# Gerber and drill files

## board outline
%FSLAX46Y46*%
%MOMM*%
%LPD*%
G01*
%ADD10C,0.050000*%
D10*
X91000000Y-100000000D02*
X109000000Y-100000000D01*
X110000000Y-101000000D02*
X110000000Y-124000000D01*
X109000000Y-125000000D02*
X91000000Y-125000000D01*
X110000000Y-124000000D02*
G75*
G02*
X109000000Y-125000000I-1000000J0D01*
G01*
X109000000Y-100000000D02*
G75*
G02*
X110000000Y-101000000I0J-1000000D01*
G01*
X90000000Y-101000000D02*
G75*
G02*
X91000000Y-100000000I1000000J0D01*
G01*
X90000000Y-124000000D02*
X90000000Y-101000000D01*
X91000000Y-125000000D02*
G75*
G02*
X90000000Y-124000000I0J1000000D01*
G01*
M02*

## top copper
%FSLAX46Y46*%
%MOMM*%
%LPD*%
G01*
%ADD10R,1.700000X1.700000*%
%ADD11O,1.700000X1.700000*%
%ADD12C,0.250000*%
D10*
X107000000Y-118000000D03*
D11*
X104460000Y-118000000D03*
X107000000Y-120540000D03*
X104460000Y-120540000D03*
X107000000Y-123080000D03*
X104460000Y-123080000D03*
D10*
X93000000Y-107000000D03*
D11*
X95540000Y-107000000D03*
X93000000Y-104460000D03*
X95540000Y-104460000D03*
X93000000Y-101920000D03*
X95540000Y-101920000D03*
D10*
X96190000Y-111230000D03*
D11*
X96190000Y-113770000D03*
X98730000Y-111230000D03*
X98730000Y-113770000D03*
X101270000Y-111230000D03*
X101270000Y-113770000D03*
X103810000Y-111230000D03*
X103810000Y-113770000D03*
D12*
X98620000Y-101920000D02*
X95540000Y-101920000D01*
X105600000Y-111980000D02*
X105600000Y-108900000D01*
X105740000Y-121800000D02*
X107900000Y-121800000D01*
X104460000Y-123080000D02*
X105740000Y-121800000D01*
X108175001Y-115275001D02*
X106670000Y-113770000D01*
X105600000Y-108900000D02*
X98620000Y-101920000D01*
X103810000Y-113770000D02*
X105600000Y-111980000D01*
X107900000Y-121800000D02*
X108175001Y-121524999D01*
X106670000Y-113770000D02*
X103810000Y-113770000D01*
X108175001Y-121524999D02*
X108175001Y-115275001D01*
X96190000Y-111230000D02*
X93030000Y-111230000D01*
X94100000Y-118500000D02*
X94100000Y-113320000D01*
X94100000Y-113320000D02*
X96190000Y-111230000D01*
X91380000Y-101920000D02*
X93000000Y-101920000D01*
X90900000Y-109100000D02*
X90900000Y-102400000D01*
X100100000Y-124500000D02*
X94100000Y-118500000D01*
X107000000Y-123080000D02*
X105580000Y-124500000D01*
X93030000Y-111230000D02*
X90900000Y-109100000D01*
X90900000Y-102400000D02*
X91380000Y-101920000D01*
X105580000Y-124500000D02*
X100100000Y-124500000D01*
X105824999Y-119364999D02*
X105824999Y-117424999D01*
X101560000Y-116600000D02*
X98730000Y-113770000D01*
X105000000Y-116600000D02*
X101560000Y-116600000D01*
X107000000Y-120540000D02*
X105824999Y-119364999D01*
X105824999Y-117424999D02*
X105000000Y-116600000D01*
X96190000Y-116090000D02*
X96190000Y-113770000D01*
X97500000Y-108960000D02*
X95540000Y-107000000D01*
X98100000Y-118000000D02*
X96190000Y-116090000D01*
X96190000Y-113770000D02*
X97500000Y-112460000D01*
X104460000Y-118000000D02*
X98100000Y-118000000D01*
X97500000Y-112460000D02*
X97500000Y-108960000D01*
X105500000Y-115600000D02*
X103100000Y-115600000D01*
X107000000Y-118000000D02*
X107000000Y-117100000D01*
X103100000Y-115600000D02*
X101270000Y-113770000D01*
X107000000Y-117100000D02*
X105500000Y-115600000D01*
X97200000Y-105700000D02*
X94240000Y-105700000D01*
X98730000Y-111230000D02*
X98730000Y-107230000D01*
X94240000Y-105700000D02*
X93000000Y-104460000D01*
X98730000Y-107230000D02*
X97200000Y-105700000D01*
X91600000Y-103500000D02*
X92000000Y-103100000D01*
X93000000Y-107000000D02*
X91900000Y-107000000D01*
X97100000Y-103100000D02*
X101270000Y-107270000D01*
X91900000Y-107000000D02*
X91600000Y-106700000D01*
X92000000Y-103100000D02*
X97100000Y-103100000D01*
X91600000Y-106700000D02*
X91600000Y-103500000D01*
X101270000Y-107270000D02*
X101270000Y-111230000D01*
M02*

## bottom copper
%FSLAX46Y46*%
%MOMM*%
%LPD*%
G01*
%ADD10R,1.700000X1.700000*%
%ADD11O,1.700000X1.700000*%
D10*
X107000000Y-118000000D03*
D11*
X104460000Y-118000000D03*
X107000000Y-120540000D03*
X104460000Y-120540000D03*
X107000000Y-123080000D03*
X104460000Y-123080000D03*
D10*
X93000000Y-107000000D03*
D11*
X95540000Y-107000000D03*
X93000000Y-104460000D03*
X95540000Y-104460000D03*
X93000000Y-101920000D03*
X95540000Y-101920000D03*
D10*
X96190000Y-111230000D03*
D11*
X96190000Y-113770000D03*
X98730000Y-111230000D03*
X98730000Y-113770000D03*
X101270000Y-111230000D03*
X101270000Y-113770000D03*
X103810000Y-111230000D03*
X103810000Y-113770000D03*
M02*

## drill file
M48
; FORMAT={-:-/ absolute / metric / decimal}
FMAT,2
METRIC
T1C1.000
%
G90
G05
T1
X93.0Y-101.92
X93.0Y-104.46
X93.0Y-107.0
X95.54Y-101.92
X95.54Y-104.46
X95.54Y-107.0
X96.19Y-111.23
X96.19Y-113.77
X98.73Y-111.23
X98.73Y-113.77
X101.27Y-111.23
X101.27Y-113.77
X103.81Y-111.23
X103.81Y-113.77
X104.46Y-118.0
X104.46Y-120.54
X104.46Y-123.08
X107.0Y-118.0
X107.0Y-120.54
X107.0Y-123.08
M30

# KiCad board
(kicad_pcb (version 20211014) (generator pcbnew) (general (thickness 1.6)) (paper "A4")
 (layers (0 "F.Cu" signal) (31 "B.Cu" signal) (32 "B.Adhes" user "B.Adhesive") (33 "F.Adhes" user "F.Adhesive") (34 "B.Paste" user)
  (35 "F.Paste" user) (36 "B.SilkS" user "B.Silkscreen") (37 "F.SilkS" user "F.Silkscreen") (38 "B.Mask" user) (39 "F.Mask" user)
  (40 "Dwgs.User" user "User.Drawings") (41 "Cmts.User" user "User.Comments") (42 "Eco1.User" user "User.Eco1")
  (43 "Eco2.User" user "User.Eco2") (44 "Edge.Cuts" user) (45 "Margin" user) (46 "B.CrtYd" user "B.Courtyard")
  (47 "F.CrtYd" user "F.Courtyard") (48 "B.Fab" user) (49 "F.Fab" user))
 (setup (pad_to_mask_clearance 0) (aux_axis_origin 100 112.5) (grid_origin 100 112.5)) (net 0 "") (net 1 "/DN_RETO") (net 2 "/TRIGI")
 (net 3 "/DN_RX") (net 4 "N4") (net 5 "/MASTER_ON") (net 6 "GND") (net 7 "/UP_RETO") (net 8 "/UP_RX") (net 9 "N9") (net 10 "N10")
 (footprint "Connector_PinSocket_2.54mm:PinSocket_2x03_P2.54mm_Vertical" (layer "F.Cu") (at 107 118)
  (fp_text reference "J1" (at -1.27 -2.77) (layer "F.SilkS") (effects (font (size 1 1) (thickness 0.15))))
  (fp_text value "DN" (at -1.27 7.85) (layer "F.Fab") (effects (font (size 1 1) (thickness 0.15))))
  (pad "1" thru_hole rect locked (at 0 0) (size 1.7 1.7) (drill 1) (layers *.Cu *.Mask) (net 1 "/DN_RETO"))
  (pad "2" thru_hole oval locked (at -2.54 0) (size 1.7 1.7) (drill 1) (layers *.Cu *.Mask) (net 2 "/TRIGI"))
  (pad "3" thru_hole oval locked (at 0 2.54) (size 1.7 1.7) (drill 1) (layers *.Cu *.Mask) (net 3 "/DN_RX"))
  (pad "4" thru_hole oval locked (at -2.54 2.54) (size 1.7 1.7) (drill 1) (layers *.Cu *.Mask) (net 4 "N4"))
  (pad "5" thru_hole oval locked (at 0 5.08) (size 1.7 1.7) (drill 1) (layers *.Cu *.Mask) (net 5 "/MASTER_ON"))
  (pad "6" thru_hole oval locked (at -2.54 5.08) (size 1.7 1.7) (drill 1) (layers *.Cu *.Mask) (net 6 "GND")))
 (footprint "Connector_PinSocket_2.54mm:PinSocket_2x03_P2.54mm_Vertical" (layer "F.Cu") (at 93 107 180)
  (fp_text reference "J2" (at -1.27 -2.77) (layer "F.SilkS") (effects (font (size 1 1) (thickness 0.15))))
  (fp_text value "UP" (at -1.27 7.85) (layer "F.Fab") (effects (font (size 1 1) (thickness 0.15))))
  (pad "1" thru_hole rect locked (at 0 0 180) (size 1.7 1.7) (drill 1) (layers *.Cu *.Mask) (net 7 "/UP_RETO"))
  (pad "2" thru_hole oval locked (at -2.54 0 180) (size 1.7 1.7) (drill 1) (layers *.Cu *.Mask) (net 2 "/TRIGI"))
  (pad "3" thru_hole oval locked (at 0 2.54 180) (size 1.7 1.7) (drill 1) (layers *.Cu *.Mask) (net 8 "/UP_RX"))
  (pad "4" thru_hole oval locked (at -2.54 2.54 180) (size 1.7 1.7) (drill 1) (layers *.Cu *.Mask) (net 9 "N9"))
  (pad "5" thru_hole oval locked (at 0 5.08 180) (size 1.7 1.7) (drill 1) (layers *.Cu *.Mask) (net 5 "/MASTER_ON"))
  (pad "6" thru_hole oval locked (at -2.54 5.08 180) (size 1.7 1.7) (drill 1) (layers *.Cu *.Mask) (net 6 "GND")))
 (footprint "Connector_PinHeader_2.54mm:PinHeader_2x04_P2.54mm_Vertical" (layer "B.Cu") (at 96.19 111.23 -90)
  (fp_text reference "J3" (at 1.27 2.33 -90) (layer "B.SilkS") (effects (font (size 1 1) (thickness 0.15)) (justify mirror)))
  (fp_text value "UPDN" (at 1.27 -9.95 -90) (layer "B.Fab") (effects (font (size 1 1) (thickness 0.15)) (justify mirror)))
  (pad "1" thru_hole rect locked (at 0 0 270) (size 1.7 1.7) (drill 1) (layers *.Cu *.Mask) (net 5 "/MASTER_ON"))
  (pad "2" thru_hole oval locked (at 2.54 0 270) (size 1.7 1.7) (drill 1) (layers *.Cu *.Mask) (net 2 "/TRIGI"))
  (pad "3" thru_hole oval locked (at 0 -2.54 270) (size 1.7 1.7) (drill 1) (layers *.Cu *.Mask) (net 8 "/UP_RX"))
  (pad "4" thru_hole oval locked (at 2.54 -2.54 270) (size 1.7 1.7) (drill 1) (layers *.Cu *.Mask) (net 3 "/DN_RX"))
  (pad "5" thru_hole oval locked (at 0 -5.08 270) (size 1.7 1.7) (drill 1) (layers *.Cu *.Mask) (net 7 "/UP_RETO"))
  (pad "6" thru_hole oval locked (at 2.54 -5.08 270) (size 1.7 1.7) (drill 1) (layers *.Cu *.Mask) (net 1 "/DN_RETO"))
  (pad "7" thru_hole oval locked (at 0 -7.62 270) (size 1.7 1.7) (drill 1) (layers *.Cu *.Mask) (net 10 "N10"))
  (pad "8" thru_hole oval locked (at 2.54 -7.62 270) (size 1.7 1.7) (drill 1) (layers *.Cu *.Mask) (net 6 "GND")))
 (gr_line (start 91 100) (end 109 100) (layer "Edge.Cuts") (width 0.05))
 (gr_line (start 110 101) (end 110 124) (layer "Edge.Cuts") (width 0.05))
 (gr_line (start 109 125) (end 91 125) (layer "Edge.Cuts") (width 0.05))
 (gr_arc (start 110 124) (mid 109.707107 124.707107) (end 109 125) (layer "Edge.Cuts") (width 0.05))
 (gr_arc (start 109 100) (mid 109.707107 100.292893) (end 110 101) (layer "Edge.Cuts") (width 0.05))
 (gr_arc (start 90 101) (mid 90.292893 100.292893) (end 91 100) (layer "Edge.Cuts") (width 0.05))
 (gr_line (start 90 124) (end 90 101) (layer "Edge.Cuts") (width 0.05))
 (gr_arc (start 91 125) (mid 90.292893 124.707107) (end 90 124) (layer "Edge.Cuts") (width 0.05))
 (segment (start 98.62 101.92) (end 95.54 101.92) (width 0.25) (layer "F.Cu") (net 6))
 (segment (start 105.6 111.98) (end 105.6 108.9) (width 0.25) (layer "F.Cu") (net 6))
 (segment (start 105.74 121.8) (end 107.9 121.8) (width 0.25) (layer "F.Cu") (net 6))
 (segment (start 104.46 123.08) (end 105.74 121.8) (width 0.25) (layer "F.Cu") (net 6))
 (segment (start 108.175001 115.275001) (end 106.67 113.77) (width 0.25) (layer "F.Cu") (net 6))
 (segment (start 105.6 108.9) (end 98.62 101.92) (width 0.25) (layer "F.Cu") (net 6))
 (segment (start 103.81 113.77) (end 105.6 111.98) (width 0.25) (layer "F.Cu") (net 6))
 (segment (start 107.9 121.8) (end 108.175001 121.524999) (width 0.25) (layer "F.Cu") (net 6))
 (segment (start 106.67 113.77) (end 103.81 113.77) (width 0.25) (layer "F.Cu") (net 6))
 (segment (start 108.175001 121.524999) (end 108.175001 115.275001) (width 0.25) (layer "F.Cu") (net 6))
 (segment (start 96.19 111.23) (end 93.03 111.23) (width 0.25) (layer "F.Cu") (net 5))
 (segment (start 94.1 118.5) (end 94.1 113.32) (width 0.25) (layer "F.Cu") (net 5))
 (segment (start 94.1 113.32) (end 96.19 111.23) (width 0.25) (layer "F.Cu") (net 5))
 (segment (start 91.38 101.92) (end 93 101.92) (width 0.25) (layer "F.Cu") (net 5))
 (segment (start 90.9 109.1) (end 90.9 102.4) (width 0.25) (layer "F.Cu") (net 5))
 (segment (start 100.1 124.5) (end 94.1 118.5) (width 0.25) (layer "F.Cu") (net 5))
 (segment (start 107 123.08) (end 105.58 124.5) (width 0.25) (layer "F.Cu") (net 5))
 (segment (start 93.03 111.23) (end 90.9 109.1) (width 0.25) (layer "F.Cu") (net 5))
 (segment (start 90.9 102.4) (end 91.38 101.92) (width 0.25) (layer "F.Cu") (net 5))
 (segment (start 105.58 124.5) (end 100.1 124.5) (width 0.25) (layer "F.Cu") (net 5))
 (segment (start 105.824999 119.364999) (end 105.824999 117.424999) (width 0.25) (layer "F.Cu") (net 3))
 (segment (start 101.56 116.6) (end 98.73 113.77) (width 0.25) (layer "F.Cu") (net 3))
 (segment (start 105 116.6) (end 101.56 116.6) (width 0.25) (layer "F.Cu") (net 3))
 (segment (start 107 120.54) (end 105.824999 119.364999) (width 0.25) (layer "F.Cu") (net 3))
 (segment (start 105.824999 117.424999) (end 105 116.6) (width 0.25) (layer "F.Cu") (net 3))
 (segment (start 96.19 116.09) (end 96.19 113.77) (width 0.25) (layer "F.Cu") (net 2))
 (segment (start 97.5 108.96) (end 95.54 107) (width 0.25) (layer "F.Cu") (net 2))
 (segment (start 98.1 118) (end 96.19 116.09) (width 0.25) (layer "F.Cu") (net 2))
 (segment (start 96.19 113.77) (end 97.5 112.46) (width 0.25) (layer "F.Cu") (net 2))
 (segment (start 104.46 118) (end 98.1 118) (width 0.25) (layer "F.Cu") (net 2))
 (segment (start 97.5 112.46) (end 97.5 108.96) (width 0.25) (layer "F.Cu") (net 2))
 (segment (start 105.5 115.6) (end 103.1 115.6) (width 0.25) (layer "F.Cu") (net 1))
 (segment (start 107 118) (end 107 117.1) (width 0.25) (layer "F.Cu") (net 1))
 (segment (start 103.1 115.6) (end 101.27 113.77) (width 0.25) (layer "F.Cu") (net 1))
 (segment (start 107 117.1) (end 105.5 115.6) (width 0.25) (layer "F.Cu") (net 1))
 (segment (start 97.2 105.7) (end 94.24 105.7) (width 0.25) (layer "F.Cu") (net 8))
 (segment (start 98.73 111.23) (end 98.73 107.23) (width 0.25) (layer "F.Cu") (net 8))
 (segment (start 94.24 105.7) (end 93 104.46) (width 0.25) (layer "F.Cu") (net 8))
 (segment (start 98.73 107.23) (end 97.2 105.7) (width 0.25) (layer "F.Cu") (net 8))
 (segment (start 91.6 103.5) (end 92 103.1) (width 0.25) (layer "F.Cu") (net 7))
 (segment (start 93 107) (end 91.9 107) (width 0.25) (layer "F.Cu") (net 7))
 (segment (start 97.1 103.1) (end 101.27 107.27) (width 0.25) (layer "F.Cu") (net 7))
 (segment (start 91.9 107) (end 91.6 106.7) (width 0.25) (layer "F.Cu") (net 7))
 (segment (start 92 103.1) (end 97.1 103.1) (width 0.25) (layer "F.Cu") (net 7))
 (segment (start 91.6 106.7) (end 91.6 103.5) (width 0.25) (layer "F.Cu") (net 7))
 (segment (start 101.27 107.27) (end 101.27 111.23) (width 0.25) (layer "F.Cu") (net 7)))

